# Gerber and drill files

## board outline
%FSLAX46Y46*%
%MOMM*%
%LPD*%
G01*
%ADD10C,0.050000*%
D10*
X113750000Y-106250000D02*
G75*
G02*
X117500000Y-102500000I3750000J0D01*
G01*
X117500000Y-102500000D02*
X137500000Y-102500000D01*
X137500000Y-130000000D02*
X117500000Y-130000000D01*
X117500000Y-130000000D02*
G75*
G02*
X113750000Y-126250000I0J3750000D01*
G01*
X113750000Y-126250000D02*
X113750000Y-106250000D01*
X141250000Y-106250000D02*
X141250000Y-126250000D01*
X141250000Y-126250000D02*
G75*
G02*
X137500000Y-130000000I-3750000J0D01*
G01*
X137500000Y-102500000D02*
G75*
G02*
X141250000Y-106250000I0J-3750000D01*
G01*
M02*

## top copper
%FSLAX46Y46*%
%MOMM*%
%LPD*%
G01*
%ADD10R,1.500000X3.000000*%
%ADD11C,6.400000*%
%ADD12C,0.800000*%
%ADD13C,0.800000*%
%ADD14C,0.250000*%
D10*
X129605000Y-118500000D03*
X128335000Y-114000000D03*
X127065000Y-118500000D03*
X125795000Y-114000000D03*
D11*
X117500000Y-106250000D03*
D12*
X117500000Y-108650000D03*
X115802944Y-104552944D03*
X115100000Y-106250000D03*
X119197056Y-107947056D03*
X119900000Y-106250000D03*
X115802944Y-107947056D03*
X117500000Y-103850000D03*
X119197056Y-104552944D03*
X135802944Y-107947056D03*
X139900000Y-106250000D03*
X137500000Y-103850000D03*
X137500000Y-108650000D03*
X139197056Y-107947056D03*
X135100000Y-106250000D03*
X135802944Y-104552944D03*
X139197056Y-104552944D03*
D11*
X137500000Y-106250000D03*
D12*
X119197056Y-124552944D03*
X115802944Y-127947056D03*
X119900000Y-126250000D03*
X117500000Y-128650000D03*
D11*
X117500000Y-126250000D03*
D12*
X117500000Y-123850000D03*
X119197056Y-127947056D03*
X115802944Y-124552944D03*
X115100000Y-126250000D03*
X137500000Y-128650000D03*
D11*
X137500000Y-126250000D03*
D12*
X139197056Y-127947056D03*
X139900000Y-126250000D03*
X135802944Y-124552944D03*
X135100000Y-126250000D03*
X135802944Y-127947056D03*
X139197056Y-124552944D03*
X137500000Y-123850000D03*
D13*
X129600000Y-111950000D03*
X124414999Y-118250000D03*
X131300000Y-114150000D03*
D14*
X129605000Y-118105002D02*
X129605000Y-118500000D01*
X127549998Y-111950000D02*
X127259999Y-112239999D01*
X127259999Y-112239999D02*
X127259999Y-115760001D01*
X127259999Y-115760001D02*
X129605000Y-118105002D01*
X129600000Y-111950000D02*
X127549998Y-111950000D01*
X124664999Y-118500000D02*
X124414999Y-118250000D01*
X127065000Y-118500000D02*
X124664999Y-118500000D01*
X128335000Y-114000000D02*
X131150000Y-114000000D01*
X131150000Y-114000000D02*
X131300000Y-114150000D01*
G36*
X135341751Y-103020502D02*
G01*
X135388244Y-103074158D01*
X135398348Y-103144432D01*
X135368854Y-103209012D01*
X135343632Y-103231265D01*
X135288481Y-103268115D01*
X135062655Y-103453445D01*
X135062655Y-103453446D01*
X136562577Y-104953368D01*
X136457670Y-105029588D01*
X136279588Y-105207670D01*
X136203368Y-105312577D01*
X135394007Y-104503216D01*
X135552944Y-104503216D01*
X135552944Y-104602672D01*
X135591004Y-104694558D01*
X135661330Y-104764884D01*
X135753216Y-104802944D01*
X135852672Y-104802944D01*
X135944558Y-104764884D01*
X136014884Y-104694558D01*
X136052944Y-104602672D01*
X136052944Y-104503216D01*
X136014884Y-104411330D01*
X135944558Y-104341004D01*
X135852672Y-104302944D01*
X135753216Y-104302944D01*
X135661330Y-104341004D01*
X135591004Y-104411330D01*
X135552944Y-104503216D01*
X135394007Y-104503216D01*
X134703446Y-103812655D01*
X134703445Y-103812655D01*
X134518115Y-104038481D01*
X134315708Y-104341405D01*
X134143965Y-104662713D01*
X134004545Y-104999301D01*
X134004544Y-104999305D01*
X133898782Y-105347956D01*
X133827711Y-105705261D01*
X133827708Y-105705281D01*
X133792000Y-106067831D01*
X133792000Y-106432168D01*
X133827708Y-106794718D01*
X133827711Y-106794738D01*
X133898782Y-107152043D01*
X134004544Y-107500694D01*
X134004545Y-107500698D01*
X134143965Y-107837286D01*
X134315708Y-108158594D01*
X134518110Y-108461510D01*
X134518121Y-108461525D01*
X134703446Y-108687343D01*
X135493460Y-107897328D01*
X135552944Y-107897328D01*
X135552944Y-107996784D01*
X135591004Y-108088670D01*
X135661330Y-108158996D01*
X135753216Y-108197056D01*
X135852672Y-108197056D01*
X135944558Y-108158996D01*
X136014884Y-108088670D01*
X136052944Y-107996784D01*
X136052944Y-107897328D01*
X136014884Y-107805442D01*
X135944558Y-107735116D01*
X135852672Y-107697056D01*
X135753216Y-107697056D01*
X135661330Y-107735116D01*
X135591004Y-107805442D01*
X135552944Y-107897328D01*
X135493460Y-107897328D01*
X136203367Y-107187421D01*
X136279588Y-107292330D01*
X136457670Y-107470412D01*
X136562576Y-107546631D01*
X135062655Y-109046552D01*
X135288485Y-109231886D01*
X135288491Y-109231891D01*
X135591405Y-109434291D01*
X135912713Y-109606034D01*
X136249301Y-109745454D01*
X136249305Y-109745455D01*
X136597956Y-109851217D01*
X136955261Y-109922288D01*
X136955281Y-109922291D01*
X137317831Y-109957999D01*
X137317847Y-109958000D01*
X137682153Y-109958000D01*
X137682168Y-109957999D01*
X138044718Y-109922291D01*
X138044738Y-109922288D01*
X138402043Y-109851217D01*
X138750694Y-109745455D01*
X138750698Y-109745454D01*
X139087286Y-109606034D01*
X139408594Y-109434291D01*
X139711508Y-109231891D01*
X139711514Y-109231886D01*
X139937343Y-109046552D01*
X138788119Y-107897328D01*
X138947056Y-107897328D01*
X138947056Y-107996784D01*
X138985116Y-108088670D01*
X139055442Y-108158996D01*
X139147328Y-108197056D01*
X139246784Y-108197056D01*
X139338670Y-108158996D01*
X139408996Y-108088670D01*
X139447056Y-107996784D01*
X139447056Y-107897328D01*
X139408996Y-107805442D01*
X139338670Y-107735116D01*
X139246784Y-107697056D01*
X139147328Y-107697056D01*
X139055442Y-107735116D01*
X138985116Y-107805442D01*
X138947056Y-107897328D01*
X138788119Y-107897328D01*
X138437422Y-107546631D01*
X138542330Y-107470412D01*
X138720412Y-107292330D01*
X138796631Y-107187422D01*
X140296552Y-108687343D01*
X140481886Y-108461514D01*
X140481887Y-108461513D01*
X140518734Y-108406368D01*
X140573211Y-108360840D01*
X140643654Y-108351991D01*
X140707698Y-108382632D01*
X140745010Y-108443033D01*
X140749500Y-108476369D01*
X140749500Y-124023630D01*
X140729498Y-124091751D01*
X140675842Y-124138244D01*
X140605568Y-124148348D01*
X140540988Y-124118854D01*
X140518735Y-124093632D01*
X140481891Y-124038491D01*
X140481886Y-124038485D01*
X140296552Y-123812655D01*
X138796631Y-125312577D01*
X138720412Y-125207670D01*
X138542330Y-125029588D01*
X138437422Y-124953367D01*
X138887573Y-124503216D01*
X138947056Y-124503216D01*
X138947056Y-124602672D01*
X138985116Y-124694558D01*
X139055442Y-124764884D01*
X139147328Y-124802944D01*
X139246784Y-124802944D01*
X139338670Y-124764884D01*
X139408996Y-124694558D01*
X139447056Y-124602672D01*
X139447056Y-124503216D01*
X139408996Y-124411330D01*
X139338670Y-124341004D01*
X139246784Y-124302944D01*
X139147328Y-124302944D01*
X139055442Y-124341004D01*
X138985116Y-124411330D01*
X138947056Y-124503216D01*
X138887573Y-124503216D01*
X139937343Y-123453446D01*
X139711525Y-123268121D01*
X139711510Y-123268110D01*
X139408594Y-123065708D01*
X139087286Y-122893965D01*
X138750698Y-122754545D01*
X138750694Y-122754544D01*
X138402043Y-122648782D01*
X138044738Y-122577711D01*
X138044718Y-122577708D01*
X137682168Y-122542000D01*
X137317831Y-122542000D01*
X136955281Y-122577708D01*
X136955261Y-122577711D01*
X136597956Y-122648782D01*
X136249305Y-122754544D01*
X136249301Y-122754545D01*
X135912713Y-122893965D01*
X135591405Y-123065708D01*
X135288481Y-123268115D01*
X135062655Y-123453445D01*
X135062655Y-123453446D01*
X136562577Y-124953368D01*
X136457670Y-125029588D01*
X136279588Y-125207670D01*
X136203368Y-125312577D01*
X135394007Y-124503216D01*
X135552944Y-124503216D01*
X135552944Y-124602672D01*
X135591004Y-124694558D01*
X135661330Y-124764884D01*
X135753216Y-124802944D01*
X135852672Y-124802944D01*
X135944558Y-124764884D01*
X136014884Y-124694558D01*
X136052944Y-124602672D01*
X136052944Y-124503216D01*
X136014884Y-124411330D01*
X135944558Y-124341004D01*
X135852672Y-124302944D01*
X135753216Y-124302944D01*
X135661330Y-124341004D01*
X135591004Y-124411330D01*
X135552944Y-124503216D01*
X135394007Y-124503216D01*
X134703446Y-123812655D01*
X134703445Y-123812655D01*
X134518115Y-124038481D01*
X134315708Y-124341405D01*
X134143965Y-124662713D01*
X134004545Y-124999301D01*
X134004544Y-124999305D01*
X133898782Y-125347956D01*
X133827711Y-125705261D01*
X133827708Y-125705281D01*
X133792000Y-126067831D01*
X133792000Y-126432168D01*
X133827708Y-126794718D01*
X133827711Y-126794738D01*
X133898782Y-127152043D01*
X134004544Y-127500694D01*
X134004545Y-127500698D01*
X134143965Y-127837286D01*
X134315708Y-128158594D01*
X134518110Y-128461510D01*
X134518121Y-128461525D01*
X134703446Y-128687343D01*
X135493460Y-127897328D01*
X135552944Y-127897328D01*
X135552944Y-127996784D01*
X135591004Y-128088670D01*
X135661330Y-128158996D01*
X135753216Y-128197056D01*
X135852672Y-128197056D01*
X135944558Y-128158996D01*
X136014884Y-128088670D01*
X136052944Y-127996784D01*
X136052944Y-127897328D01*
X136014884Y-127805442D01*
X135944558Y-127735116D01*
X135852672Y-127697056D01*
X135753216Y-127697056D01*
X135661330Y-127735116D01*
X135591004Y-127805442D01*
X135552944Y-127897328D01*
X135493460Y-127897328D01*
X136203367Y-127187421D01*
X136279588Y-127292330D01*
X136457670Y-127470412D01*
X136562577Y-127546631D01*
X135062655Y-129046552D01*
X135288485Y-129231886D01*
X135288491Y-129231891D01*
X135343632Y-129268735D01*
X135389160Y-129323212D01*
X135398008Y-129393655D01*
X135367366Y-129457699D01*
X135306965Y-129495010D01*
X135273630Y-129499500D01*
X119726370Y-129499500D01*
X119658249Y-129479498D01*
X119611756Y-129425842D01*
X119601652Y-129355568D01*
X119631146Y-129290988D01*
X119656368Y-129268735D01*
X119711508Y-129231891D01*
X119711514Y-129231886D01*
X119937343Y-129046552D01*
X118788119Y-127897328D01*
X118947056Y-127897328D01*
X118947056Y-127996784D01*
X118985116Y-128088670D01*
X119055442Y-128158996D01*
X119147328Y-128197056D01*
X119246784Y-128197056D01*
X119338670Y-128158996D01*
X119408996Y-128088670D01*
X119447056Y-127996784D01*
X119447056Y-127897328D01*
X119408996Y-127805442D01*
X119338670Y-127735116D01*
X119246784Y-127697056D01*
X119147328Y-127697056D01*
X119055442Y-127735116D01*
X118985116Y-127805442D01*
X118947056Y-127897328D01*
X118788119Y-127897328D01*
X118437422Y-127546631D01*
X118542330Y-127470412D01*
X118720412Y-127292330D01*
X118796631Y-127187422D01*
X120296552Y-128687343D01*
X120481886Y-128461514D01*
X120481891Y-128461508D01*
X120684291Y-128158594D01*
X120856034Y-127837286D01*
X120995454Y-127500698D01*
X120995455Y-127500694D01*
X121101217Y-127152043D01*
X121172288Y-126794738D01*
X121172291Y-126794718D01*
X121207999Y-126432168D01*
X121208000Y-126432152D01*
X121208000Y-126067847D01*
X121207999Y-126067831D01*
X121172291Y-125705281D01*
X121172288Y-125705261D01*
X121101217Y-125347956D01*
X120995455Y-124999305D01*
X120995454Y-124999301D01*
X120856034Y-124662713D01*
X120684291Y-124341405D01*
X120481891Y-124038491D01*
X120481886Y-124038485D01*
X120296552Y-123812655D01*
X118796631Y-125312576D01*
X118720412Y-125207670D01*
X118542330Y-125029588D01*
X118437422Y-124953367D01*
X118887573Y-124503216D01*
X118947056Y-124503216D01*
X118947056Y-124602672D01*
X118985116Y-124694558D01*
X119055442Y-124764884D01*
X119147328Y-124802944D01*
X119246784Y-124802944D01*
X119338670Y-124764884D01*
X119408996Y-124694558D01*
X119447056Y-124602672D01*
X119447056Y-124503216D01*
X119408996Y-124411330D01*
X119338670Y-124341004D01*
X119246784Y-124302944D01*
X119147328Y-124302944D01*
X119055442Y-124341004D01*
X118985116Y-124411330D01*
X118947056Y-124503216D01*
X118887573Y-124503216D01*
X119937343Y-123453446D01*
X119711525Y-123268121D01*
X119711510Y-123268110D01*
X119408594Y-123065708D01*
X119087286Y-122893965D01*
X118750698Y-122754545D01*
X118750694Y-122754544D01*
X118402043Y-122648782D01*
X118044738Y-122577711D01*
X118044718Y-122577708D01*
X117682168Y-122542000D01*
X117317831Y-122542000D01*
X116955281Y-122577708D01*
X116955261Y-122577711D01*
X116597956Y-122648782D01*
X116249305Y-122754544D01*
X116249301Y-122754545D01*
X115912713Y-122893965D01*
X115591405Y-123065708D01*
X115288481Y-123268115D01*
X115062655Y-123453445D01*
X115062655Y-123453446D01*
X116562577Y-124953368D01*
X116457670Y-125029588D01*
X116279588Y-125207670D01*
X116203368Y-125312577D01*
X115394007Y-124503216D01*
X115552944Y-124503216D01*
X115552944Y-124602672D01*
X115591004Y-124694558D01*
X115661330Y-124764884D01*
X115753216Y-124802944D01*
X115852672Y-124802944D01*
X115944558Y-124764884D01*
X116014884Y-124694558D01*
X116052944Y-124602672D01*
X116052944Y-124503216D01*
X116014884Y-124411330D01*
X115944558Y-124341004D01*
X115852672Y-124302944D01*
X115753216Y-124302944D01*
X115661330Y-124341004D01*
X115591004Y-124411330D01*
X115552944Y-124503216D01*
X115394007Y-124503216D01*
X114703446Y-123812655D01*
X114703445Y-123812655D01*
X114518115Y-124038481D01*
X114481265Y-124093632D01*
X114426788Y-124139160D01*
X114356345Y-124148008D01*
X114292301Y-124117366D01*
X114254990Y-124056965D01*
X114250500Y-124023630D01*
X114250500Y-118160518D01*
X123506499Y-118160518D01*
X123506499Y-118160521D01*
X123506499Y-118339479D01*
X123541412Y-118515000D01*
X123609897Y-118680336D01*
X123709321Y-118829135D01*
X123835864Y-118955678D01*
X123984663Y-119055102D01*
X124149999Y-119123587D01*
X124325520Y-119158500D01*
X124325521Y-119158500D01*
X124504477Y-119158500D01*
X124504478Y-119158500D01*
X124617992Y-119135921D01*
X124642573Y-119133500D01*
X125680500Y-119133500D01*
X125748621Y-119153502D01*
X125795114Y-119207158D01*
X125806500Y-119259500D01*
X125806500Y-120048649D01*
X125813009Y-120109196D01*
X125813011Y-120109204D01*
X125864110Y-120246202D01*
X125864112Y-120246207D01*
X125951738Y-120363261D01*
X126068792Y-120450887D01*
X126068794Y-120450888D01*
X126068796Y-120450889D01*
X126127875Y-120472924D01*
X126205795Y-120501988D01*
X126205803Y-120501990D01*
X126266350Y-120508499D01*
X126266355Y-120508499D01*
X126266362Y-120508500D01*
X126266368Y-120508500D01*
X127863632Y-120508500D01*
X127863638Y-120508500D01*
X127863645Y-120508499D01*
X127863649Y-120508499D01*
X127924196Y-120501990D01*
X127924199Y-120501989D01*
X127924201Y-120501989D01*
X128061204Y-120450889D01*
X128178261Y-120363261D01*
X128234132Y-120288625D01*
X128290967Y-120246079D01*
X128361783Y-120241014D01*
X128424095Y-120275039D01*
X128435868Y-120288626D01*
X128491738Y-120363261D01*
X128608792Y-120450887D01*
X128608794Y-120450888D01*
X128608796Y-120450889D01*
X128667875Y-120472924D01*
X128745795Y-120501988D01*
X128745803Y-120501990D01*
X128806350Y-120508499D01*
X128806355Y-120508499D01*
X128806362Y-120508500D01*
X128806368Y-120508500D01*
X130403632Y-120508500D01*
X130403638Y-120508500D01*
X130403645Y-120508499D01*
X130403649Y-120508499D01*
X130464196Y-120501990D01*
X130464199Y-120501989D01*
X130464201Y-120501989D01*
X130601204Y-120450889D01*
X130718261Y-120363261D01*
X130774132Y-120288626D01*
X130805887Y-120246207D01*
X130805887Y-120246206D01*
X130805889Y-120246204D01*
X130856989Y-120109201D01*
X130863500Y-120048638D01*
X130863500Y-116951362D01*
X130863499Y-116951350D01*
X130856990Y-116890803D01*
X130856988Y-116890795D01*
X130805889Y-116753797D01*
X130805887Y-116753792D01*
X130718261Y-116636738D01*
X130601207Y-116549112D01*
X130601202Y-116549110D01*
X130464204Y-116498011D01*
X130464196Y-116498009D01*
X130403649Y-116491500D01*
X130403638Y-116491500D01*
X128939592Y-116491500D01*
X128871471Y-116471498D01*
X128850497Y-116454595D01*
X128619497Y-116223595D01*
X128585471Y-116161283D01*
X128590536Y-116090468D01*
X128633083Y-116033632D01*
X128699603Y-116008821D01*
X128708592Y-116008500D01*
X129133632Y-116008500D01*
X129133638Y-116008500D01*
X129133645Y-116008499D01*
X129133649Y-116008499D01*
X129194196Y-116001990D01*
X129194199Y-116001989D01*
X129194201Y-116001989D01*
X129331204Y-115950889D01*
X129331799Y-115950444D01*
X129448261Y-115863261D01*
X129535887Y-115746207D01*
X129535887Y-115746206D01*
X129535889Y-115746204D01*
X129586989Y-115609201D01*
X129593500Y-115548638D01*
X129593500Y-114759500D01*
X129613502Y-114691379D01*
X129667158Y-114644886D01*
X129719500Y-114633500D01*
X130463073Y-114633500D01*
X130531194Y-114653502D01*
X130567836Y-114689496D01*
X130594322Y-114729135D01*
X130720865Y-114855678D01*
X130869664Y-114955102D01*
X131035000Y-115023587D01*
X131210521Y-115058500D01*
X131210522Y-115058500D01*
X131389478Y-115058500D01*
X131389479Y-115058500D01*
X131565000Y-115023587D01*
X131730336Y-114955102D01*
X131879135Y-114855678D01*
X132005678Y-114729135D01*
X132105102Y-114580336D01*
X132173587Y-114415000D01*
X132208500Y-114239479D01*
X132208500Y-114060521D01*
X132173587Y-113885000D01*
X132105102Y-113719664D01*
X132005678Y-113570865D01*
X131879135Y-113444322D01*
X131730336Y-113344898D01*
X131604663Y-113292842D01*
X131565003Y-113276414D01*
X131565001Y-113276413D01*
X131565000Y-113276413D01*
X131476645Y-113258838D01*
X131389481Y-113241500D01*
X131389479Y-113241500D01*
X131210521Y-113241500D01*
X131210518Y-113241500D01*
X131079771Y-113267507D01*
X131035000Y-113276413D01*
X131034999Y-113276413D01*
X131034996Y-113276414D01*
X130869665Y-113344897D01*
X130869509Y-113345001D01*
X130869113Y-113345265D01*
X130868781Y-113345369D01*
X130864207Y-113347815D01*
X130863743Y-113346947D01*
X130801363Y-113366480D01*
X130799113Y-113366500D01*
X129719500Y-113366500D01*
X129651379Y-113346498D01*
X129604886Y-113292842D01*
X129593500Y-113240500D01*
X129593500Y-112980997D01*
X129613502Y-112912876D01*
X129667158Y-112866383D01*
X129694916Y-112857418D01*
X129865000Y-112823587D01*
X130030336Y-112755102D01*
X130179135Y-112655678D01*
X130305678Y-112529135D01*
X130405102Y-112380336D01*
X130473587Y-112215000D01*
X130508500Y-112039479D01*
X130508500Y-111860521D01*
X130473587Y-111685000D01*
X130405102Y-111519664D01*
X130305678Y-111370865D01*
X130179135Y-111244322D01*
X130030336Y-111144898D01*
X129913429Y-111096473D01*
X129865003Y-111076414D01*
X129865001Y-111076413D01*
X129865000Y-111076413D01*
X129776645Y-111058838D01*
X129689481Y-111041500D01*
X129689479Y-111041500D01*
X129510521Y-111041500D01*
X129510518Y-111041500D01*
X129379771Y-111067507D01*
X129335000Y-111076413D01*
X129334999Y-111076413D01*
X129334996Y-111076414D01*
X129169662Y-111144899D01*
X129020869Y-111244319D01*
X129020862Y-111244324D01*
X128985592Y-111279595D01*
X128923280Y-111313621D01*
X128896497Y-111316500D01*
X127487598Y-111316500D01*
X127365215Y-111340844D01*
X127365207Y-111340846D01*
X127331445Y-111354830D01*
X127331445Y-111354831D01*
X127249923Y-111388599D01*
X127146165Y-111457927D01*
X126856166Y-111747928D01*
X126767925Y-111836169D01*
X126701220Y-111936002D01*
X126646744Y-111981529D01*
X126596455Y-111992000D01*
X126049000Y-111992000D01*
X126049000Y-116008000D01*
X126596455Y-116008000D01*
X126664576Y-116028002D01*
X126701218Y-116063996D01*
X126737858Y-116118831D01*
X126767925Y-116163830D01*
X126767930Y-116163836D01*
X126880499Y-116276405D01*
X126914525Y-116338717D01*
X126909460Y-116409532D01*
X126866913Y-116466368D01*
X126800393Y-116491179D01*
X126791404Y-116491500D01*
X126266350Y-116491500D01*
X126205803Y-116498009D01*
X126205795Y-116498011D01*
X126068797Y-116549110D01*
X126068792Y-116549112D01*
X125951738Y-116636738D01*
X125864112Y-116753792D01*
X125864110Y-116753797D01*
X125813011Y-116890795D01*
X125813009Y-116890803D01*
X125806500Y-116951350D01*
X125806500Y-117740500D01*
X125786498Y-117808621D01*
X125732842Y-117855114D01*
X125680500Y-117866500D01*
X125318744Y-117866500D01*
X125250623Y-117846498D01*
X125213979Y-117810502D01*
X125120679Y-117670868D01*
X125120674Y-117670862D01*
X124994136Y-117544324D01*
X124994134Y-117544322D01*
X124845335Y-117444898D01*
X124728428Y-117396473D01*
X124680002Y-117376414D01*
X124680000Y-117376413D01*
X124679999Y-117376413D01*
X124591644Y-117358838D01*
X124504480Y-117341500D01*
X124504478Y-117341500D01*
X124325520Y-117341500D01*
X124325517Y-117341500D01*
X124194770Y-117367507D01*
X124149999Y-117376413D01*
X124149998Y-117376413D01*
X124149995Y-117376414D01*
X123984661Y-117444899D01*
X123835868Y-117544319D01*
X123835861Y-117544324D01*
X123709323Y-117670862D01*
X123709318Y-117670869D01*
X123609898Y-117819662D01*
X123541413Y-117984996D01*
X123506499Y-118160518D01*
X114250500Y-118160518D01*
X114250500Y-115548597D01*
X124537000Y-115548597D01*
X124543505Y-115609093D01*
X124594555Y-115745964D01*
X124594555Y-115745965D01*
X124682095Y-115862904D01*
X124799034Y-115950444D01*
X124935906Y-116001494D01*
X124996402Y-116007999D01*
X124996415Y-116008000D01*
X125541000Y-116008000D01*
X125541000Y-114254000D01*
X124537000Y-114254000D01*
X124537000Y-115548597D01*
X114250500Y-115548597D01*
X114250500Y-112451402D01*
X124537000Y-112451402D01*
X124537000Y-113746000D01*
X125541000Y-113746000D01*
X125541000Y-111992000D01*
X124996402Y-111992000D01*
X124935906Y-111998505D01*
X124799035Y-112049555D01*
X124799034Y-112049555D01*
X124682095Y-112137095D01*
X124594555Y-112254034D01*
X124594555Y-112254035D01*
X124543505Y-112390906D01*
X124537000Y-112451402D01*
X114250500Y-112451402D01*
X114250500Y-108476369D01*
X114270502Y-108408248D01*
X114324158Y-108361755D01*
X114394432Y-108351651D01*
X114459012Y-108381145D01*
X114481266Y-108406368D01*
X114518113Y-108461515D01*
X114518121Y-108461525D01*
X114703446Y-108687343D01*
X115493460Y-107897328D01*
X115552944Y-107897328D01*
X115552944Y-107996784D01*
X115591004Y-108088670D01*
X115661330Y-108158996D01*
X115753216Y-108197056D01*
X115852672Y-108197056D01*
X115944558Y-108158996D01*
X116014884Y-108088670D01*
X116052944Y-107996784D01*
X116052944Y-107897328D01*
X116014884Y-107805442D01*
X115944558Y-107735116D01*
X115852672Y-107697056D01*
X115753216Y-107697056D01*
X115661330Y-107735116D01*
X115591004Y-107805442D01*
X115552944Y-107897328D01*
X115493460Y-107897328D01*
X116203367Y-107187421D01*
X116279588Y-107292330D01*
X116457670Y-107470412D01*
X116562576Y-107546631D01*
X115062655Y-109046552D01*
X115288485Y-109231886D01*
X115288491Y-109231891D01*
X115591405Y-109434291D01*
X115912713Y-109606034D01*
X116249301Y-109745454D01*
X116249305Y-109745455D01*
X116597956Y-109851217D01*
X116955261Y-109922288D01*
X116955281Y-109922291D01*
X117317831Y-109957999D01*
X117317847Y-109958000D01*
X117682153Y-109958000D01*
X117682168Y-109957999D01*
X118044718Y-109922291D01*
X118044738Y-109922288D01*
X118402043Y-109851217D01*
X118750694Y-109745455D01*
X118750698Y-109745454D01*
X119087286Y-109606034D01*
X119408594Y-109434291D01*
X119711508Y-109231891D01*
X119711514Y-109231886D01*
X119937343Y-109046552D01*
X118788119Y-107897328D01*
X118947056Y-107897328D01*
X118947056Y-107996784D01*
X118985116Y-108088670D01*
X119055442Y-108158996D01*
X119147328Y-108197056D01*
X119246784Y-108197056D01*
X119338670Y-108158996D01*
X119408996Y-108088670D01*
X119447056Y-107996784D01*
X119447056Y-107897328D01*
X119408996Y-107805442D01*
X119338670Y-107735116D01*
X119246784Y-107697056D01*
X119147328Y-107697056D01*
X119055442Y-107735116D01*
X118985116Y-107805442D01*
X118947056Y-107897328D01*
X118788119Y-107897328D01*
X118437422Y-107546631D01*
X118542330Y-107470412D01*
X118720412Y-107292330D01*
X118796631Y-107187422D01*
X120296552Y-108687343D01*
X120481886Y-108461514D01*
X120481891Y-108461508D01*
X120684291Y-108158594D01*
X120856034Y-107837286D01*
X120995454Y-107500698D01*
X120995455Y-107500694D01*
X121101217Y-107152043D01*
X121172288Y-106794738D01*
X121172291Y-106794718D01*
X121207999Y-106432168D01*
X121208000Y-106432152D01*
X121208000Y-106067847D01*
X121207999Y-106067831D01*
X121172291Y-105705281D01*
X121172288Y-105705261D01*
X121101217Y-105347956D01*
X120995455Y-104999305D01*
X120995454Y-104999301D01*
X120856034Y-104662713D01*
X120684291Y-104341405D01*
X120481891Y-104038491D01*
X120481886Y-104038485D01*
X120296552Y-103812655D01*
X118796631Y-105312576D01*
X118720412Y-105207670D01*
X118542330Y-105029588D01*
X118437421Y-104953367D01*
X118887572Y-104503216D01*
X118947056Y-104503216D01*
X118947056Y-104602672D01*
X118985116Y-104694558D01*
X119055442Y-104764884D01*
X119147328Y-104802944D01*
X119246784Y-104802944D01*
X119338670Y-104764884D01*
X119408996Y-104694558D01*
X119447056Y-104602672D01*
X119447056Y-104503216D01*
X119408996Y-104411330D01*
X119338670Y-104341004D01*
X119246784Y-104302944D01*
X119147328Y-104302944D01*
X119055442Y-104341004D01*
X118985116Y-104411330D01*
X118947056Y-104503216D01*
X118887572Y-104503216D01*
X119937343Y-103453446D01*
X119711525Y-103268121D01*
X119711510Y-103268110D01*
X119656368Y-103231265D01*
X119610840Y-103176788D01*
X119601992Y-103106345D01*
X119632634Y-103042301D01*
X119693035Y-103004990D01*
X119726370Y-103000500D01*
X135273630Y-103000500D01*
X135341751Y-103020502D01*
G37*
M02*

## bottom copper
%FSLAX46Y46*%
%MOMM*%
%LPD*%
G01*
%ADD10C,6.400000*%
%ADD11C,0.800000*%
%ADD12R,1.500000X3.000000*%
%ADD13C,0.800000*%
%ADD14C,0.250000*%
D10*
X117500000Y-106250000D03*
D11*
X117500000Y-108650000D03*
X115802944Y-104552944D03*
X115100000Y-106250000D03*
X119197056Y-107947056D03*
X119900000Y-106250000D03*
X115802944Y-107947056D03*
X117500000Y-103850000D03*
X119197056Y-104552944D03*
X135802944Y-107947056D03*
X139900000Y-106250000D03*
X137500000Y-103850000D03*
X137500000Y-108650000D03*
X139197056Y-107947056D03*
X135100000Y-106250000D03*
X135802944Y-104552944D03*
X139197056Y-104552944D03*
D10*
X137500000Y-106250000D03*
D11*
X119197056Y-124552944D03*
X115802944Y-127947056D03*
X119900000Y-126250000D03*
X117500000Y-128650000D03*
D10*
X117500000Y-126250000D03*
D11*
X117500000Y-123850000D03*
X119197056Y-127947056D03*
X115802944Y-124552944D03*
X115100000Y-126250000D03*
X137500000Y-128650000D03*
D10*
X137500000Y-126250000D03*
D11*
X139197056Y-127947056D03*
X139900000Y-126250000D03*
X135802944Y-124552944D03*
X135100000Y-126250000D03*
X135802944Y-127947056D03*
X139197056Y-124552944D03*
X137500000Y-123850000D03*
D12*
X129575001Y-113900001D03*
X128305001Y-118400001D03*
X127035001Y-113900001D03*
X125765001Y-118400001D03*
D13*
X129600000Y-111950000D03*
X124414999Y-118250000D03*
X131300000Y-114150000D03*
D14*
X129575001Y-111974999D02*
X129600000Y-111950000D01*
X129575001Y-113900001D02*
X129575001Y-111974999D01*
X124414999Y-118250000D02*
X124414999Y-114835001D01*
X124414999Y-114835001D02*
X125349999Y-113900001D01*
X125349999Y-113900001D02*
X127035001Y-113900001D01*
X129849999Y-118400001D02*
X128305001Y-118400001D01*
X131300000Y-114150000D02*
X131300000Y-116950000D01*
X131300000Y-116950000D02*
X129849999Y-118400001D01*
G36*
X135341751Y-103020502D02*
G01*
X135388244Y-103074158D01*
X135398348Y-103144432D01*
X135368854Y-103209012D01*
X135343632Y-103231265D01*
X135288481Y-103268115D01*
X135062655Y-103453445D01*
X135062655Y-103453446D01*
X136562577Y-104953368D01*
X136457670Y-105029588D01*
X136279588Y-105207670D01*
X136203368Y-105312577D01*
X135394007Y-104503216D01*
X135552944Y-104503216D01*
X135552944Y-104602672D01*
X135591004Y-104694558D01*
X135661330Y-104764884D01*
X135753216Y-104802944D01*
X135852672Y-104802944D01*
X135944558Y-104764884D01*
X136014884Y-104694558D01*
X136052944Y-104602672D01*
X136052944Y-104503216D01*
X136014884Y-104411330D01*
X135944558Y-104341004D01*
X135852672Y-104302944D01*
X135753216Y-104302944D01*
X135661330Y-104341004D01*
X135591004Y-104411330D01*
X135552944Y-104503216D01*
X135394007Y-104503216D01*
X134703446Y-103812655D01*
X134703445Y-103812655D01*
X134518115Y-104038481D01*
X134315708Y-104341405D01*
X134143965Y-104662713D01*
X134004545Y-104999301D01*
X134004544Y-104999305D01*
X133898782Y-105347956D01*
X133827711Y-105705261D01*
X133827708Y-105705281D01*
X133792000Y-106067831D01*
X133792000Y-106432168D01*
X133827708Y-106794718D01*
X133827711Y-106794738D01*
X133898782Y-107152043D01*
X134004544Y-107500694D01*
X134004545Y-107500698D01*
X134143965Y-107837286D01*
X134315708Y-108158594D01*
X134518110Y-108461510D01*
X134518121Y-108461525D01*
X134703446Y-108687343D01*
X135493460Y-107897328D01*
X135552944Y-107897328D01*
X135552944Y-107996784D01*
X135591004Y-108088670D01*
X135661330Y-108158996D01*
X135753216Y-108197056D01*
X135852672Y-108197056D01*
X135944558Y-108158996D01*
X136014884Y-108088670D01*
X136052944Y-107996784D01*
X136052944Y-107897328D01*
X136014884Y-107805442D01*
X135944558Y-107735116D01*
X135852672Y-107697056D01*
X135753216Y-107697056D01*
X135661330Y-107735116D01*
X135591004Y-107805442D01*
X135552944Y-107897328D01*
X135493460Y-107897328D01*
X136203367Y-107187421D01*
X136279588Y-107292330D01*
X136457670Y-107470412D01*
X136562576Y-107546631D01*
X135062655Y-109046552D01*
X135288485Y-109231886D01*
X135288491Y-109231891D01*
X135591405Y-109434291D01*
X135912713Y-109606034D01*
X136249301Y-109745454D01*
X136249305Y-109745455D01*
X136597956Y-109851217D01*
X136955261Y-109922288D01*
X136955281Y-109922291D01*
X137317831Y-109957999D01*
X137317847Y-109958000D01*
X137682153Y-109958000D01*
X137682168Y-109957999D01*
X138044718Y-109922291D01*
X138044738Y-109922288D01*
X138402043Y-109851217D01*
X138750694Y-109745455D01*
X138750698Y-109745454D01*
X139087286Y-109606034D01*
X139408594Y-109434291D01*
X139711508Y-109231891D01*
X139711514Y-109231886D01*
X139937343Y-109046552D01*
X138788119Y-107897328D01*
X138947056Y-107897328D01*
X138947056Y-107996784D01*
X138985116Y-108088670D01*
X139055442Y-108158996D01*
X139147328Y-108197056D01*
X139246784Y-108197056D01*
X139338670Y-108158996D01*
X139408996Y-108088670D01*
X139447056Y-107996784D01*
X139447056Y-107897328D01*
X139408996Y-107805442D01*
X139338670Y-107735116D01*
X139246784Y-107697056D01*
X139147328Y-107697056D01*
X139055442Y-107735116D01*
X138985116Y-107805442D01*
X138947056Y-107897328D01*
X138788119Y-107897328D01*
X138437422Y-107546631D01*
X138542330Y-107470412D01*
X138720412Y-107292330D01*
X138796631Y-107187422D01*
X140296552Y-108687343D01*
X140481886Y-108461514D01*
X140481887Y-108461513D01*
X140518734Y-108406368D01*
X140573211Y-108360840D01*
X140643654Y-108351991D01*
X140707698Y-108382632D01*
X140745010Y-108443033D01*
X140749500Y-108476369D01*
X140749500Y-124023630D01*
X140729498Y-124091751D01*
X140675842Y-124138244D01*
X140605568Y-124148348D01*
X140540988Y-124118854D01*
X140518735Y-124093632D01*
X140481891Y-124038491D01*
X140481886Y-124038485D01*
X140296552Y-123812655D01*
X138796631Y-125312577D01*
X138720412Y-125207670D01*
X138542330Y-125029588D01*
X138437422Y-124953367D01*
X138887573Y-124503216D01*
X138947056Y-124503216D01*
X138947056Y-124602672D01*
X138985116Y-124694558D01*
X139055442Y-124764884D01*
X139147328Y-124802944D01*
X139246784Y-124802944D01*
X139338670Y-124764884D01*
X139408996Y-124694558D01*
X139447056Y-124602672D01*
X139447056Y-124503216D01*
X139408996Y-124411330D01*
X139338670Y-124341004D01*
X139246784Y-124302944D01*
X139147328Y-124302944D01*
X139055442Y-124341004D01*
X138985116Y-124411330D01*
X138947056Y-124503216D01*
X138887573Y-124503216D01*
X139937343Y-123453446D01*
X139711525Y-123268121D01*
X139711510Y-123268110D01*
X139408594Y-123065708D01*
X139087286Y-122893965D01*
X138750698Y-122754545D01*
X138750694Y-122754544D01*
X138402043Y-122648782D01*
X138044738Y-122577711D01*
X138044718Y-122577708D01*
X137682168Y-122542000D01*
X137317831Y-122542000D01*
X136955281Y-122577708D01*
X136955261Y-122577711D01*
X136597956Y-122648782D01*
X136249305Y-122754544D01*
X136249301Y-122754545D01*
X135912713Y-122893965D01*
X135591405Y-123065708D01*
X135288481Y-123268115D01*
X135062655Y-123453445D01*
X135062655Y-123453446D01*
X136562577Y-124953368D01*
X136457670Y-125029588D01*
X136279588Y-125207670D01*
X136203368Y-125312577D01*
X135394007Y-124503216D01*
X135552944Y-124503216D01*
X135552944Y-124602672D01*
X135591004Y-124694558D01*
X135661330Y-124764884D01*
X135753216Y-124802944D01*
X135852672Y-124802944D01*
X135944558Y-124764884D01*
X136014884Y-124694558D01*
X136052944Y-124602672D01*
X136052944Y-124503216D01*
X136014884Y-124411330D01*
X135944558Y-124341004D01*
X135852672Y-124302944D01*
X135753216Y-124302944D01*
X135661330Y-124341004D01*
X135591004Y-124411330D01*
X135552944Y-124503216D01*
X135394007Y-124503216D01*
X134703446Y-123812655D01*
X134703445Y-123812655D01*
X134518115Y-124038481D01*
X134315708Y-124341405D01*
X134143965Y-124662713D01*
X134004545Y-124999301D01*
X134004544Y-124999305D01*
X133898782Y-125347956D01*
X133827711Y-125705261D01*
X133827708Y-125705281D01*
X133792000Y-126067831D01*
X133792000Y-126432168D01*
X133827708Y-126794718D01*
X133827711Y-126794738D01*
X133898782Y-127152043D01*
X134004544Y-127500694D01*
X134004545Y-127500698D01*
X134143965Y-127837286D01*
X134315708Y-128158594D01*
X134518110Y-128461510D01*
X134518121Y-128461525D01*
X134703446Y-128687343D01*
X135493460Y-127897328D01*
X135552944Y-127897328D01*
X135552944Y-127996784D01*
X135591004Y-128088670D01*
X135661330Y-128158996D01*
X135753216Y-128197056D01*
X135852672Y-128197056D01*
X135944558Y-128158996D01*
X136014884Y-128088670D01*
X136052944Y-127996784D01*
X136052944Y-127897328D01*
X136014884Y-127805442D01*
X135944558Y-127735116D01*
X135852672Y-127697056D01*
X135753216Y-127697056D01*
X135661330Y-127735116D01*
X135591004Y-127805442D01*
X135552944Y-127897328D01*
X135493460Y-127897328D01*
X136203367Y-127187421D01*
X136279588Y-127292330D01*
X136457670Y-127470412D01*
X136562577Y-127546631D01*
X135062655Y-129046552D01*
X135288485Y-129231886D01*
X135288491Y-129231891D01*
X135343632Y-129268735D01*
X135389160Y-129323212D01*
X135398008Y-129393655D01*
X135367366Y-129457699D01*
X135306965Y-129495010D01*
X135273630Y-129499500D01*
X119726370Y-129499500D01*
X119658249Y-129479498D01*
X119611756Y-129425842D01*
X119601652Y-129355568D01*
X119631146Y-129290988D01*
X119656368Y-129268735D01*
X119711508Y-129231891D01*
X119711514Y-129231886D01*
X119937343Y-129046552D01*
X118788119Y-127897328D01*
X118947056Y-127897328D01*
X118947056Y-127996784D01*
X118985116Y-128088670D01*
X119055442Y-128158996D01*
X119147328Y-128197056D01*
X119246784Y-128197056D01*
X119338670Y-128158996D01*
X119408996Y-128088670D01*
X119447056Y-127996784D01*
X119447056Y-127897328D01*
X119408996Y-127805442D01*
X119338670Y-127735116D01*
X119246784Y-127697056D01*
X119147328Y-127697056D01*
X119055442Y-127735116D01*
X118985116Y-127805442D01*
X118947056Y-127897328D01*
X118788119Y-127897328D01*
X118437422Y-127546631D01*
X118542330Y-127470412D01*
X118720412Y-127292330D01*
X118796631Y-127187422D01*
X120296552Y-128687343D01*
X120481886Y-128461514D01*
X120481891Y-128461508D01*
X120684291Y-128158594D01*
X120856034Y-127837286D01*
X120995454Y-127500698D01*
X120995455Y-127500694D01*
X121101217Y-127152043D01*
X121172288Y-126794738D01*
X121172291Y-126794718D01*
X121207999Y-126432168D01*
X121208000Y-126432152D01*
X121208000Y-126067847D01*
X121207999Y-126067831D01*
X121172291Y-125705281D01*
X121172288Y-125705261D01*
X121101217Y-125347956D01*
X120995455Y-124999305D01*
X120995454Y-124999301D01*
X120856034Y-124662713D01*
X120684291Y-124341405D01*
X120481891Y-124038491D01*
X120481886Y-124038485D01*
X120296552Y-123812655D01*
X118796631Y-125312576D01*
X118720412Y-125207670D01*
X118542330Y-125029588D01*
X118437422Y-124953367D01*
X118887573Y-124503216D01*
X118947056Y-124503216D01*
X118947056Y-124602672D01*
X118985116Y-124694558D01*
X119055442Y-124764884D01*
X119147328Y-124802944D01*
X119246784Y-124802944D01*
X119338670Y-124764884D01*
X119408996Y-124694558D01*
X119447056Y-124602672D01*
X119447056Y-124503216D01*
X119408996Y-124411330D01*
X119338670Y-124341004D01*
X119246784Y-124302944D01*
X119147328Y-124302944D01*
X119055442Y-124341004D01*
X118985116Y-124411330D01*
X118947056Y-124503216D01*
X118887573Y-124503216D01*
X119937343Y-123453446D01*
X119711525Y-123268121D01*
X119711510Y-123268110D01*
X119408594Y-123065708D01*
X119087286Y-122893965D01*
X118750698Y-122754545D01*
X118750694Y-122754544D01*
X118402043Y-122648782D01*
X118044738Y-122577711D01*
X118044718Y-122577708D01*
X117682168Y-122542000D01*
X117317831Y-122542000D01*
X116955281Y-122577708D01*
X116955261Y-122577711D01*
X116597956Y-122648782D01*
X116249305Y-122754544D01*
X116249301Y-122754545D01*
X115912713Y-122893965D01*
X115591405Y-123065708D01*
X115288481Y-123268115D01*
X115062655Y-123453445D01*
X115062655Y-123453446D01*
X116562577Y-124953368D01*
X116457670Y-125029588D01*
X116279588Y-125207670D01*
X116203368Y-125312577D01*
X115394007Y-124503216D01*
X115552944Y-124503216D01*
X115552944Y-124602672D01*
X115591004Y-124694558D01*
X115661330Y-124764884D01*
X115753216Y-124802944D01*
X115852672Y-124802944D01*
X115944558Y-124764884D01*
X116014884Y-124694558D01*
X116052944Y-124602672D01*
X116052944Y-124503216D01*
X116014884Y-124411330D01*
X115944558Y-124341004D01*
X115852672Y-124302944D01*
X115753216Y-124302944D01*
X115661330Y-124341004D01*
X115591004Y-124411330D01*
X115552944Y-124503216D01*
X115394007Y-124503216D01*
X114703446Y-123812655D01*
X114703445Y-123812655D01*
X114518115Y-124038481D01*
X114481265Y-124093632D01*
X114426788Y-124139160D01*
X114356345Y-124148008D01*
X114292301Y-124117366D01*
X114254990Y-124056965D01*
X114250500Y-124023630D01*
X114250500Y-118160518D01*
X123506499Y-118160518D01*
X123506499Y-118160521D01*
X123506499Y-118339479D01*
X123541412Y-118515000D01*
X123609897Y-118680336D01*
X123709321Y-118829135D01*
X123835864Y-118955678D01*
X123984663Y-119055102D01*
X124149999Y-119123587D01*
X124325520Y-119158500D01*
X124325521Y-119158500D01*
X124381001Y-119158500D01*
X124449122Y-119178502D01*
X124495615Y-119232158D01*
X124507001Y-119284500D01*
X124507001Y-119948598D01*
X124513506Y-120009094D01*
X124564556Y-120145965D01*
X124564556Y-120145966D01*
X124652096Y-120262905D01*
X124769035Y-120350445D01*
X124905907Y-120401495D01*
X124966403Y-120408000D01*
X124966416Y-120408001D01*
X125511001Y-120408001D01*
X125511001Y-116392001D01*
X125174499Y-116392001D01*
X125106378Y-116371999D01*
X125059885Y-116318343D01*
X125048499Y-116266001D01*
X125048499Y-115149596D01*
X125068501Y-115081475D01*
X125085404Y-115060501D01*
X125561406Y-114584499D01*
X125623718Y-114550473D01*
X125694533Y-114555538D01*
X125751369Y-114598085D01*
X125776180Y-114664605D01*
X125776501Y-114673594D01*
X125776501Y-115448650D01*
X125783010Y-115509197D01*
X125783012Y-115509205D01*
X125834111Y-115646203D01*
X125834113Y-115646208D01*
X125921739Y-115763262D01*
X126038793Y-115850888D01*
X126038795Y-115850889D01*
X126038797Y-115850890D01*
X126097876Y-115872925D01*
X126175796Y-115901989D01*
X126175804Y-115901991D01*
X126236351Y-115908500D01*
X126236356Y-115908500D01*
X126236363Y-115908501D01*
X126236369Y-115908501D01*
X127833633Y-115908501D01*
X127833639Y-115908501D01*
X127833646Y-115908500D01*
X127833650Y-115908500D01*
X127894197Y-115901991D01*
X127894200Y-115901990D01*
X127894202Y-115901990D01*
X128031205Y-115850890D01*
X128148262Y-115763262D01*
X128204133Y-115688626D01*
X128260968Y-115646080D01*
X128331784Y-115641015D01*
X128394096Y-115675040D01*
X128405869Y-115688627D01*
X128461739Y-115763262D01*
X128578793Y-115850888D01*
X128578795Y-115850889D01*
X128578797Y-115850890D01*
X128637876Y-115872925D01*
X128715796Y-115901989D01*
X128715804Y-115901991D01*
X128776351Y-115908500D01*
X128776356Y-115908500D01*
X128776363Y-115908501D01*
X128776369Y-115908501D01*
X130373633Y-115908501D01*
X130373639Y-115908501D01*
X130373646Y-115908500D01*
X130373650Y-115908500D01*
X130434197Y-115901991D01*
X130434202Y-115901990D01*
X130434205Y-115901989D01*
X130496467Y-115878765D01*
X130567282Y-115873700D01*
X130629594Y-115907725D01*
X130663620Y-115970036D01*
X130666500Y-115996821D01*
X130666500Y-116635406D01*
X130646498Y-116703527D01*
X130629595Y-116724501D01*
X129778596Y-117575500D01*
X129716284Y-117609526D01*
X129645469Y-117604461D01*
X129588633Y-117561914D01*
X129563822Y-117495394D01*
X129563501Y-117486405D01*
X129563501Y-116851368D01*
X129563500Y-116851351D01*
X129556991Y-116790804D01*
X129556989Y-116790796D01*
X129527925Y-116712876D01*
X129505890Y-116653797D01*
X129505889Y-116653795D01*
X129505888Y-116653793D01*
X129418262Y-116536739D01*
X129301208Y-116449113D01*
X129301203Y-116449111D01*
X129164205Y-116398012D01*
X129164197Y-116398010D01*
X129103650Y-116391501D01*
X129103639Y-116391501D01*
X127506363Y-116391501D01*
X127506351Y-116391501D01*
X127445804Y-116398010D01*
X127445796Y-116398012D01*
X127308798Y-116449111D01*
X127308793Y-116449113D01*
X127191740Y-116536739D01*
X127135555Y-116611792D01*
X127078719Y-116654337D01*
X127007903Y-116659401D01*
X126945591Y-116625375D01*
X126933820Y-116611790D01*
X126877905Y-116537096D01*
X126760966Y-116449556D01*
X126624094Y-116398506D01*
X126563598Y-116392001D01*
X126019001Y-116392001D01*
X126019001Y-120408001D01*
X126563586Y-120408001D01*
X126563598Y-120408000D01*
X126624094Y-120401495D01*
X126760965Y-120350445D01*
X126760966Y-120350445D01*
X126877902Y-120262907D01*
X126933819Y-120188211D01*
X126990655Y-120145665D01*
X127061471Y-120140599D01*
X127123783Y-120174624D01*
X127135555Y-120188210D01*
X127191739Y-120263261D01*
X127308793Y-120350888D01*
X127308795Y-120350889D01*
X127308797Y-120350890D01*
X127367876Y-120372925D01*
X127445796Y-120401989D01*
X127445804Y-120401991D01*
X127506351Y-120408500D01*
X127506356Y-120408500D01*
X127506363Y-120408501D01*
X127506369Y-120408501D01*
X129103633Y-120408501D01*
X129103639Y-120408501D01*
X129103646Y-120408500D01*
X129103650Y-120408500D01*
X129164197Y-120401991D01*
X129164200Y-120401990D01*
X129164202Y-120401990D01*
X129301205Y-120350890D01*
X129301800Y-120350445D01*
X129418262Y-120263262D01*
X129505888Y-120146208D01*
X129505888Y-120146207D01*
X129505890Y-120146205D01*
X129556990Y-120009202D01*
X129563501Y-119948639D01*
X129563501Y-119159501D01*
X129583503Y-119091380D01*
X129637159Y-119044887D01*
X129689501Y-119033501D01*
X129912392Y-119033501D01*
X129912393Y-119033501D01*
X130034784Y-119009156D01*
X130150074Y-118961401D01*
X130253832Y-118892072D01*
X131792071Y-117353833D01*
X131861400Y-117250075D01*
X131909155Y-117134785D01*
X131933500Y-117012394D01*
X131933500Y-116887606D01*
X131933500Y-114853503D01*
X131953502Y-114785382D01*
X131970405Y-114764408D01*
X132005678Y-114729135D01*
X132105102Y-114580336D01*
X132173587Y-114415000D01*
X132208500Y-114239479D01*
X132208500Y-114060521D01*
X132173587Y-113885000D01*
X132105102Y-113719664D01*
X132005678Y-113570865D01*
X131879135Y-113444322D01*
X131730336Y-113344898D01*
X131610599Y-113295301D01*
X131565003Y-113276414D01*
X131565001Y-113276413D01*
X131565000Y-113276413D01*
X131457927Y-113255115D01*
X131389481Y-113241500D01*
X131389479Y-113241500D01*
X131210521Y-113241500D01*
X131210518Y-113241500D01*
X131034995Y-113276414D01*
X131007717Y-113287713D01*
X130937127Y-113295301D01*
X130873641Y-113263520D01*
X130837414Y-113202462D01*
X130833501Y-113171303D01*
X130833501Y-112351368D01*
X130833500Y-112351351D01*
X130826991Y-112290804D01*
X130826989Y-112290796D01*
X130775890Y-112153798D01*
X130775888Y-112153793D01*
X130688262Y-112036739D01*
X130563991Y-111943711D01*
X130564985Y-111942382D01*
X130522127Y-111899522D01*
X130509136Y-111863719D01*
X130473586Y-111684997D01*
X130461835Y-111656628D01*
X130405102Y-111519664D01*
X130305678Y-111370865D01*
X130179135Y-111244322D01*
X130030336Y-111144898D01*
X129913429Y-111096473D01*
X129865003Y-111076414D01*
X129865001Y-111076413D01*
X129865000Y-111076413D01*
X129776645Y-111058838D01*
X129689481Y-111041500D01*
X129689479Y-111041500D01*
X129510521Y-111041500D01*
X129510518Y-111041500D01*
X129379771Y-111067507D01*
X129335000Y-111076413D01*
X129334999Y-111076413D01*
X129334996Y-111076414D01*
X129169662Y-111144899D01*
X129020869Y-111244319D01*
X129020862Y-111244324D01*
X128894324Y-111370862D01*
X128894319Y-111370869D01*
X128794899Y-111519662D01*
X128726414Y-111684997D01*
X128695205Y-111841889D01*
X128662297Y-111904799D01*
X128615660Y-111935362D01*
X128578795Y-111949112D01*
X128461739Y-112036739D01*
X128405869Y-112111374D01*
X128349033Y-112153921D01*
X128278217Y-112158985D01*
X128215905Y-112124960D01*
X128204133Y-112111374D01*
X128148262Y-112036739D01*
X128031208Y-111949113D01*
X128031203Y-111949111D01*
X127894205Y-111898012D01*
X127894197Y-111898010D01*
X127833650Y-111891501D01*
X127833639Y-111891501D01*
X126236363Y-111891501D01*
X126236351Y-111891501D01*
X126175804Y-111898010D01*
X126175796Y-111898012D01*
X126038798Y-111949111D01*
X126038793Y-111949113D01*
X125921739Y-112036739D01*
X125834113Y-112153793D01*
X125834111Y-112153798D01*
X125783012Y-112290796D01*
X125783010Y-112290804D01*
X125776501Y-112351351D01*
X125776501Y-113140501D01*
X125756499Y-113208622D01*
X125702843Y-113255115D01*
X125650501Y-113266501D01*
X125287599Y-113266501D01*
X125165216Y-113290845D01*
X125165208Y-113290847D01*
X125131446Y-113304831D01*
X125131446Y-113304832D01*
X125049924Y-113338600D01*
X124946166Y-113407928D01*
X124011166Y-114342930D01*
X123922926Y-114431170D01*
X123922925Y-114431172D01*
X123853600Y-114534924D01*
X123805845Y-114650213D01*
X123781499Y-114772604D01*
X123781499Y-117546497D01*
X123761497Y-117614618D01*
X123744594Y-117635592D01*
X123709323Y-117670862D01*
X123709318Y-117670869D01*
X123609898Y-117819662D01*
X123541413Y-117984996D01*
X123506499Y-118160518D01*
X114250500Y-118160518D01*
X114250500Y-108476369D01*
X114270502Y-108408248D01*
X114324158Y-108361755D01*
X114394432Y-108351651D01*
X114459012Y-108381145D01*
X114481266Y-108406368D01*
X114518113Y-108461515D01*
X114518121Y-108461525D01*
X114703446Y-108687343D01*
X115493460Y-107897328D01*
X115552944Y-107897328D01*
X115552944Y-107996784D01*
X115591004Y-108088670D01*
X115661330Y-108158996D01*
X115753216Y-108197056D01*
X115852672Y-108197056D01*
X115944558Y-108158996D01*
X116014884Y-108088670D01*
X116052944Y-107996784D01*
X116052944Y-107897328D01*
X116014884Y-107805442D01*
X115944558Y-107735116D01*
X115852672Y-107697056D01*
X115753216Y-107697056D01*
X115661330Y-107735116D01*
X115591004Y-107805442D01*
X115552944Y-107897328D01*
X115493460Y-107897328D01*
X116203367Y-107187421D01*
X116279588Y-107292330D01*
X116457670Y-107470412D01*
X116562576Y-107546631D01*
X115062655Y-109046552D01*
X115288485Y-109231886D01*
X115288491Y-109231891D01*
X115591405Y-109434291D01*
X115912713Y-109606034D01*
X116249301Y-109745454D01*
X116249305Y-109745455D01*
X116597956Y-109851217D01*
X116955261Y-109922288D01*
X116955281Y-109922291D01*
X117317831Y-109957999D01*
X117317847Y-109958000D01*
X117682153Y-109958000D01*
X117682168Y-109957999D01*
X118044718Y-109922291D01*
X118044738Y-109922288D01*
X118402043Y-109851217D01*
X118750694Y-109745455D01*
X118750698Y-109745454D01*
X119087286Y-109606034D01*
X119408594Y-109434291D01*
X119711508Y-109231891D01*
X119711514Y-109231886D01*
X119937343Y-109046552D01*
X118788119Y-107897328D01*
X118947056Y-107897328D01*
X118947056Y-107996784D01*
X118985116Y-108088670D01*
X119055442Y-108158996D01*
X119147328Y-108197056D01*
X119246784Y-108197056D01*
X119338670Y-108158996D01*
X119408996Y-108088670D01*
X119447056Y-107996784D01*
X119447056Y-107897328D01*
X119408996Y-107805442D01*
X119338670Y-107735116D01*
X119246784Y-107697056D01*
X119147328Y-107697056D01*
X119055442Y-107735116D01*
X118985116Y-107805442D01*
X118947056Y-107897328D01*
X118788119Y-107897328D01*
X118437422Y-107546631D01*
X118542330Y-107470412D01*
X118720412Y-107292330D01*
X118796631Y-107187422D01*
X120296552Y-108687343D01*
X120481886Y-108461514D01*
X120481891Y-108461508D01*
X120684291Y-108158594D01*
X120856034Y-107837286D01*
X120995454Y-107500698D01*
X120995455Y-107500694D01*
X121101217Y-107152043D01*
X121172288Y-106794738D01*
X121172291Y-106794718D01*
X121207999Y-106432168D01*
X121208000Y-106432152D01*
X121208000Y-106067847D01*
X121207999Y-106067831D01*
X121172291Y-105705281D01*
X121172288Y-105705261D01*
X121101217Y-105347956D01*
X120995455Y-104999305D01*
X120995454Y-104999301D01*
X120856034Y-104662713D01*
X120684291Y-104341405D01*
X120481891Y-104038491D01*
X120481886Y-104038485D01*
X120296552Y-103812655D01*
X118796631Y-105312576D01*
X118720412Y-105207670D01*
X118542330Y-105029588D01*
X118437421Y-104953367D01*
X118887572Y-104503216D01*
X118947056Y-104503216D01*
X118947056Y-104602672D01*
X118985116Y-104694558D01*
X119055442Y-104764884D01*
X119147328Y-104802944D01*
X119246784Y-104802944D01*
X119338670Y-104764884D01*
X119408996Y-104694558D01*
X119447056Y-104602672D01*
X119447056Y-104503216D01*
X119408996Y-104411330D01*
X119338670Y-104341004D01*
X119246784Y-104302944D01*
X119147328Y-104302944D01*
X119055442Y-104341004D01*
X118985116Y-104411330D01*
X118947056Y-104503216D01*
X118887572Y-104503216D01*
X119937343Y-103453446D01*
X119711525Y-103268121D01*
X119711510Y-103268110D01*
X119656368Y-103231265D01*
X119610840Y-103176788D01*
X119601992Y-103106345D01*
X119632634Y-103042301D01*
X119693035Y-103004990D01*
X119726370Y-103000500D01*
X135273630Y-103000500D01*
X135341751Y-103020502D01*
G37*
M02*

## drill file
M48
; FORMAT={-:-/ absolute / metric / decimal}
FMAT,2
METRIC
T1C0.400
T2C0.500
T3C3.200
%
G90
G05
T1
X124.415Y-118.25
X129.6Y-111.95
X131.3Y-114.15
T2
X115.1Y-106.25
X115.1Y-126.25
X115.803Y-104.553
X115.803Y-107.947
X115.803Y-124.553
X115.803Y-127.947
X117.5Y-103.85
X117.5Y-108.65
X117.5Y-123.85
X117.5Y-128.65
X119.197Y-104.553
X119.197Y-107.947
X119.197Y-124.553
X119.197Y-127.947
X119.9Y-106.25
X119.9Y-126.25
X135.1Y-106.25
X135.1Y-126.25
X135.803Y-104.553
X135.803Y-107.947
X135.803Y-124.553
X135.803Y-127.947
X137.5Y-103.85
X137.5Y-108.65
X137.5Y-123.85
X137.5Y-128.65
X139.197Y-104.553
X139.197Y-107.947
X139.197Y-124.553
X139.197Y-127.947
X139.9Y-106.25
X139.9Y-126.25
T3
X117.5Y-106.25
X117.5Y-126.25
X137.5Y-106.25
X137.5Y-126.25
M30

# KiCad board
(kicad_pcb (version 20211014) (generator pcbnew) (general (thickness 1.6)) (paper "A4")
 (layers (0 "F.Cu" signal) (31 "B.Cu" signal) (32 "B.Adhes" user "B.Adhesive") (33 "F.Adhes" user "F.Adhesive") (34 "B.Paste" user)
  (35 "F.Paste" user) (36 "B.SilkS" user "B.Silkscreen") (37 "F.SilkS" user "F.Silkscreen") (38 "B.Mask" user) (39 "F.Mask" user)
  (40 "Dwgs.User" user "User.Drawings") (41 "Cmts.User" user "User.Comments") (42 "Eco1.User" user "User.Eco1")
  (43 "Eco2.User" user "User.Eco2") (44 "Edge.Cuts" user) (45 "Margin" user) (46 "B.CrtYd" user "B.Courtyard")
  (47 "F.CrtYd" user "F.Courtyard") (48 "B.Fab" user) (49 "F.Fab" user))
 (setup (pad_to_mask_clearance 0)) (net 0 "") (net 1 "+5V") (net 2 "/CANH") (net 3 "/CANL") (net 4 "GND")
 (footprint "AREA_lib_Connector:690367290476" (layer "F.Cu") (at 127.7 116.25)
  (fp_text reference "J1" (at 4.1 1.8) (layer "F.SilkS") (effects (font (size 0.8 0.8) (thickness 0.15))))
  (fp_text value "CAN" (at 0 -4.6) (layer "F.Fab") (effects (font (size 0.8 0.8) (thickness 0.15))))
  (pad "1" smd rect locked (at 1.905 2.25) (size 1.5 3) (layers "F.Cu" "F.Paste" "F.Mask") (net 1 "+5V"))
  (pad "2" smd rect locked (at 0.635 -2.25) (size 1.5 3) (layers "F.Cu" "F.Paste" "F.Mask") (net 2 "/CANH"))
  (pad "3" smd rect locked (at -0.635 2.25) (size 1.5 3) (layers "F.Cu" "F.Paste" "F.Mask") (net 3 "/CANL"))
  (pad "4" smd rect locked (at -1.905 -2.25) (size 1.5 3) (layers "F.Cu" "F.Paste" "F.Mask") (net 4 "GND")))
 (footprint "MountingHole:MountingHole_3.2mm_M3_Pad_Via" (layer "F.Cu") (at 117.5 106.25)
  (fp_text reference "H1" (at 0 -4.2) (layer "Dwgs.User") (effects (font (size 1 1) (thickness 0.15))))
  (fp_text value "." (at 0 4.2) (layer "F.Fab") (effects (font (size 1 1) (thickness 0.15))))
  (pad "1" thru_hole circle locked (at 0 0) (size 6.4 6.4) (drill 3.2) (layers *.Cu *.Mask) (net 4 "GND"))
  (pad "1" thru_hole circle locked (at 0 2.4) (size 0.8 0.8) (drill 0.5) (layers *.Cu *.Mask) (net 4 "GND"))
  (pad "1" thru_hole circle locked (at -1.697056 -1.697056) (size 0.8 0.8) (drill 0.5) (layers *.Cu *.Mask) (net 4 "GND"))
  (pad "1" thru_hole circle locked (at -2.4 0) (size 0.8 0.8) (drill 0.5) (layers *.Cu *.Mask) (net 4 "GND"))
  (pad "1" thru_hole circle locked (at 1.697056 1.697056) (size 0.8 0.8) (drill 0.5) (layers *.Cu *.Mask) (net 4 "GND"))
  (pad "1" thru_hole circle locked (at 2.4 0) (size 0.8 0.8) (drill 0.5) (layers *.Cu *.Mask) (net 4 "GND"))
  (pad "1" thru_hole circle locked (at -1.697056 1.697056) (size 0.8 0.8) (drill 0.5) (layers *.Cu *.Mask) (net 4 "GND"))
  (pad "1" thru_hole circle locked (at 0 -2.4) (size 0.8 0.8) (drill 0.5) (layers *.Cu *.Mask) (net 4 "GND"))
  (pad "1" thru_hole circle locked (at 1.697056 -1.697056) (size 0.8 0.8) (drill 0.5) (layers *.Cu *.Mask) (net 4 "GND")))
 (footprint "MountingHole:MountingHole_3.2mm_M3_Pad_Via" (layer "F.Cu") (at 137.5 106.25)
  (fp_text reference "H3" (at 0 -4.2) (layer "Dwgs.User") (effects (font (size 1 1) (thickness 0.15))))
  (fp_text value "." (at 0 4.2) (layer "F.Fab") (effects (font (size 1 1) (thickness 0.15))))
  (pad "1" thru_hole circle locked (at -1.697056 1.697056) (size 0.8 0.8) (drill 0.5) (layers *.Cu *.Mask) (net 4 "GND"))
  (pad "1" thru_hole circle locked (at 2.4 0) (size 0.8 0.8) (drill 0.5) (layers *.Cu *.Mask) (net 4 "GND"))
  (pad "1" thru_hole circle locked (at 0 -2.4) (size 0.8 0.8) (drill 0.5) (layers *.Cu *.Mask) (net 4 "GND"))
  (pad "1" thru_hole circle locked (at 0 2.4) (size 0.8 0.8) (drill 0.5) (layers *.Cu *.Mask) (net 4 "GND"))
  (pad "1" thru_hole circle locked (at 1.697056 1.697056) (size 0.8 0.8) (drill 0.5) (layers *.Cu *.Mask) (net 4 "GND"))
  (pad "1" thru_hole circle locked (at -2.4 0) (size 0.8 0.8) (drill 0.5) (layers *.Cu *.Mask) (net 4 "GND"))
  (pad "1" thru_hole circle locked (at -1.697056 -1.697056) (size 0.8 0.8) (drill 0.5) (layers *.Cu *.Mask) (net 4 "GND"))
  (pad "1" thru_hole circle locked (at 1.697056 -1.697056) (size 0.8 0.8) (drill 0.5) (layers *.Cu *.Mask) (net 4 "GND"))
  (pad "1" thru_hole circle locked (at 0 0) (size 6.4 6.4) (drill 3.2) (layers *.Cu *.Mask) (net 4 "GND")))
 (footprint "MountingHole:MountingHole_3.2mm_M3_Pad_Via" (layer "F.Cu") (at 117.5 126.25)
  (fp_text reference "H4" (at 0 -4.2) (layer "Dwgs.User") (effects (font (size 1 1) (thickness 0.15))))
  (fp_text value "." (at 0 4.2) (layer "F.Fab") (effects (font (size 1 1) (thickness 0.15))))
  (pad "1" thru_hole circle locked (at 1.697056 -1.697056) (size 0.8 0.8) (drill 0.5) (layers *.Cu *.Mask) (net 4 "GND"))
  (pad "1" thru_hole circle locked (at -1.697056 1.697056) (size 0.8 0.8) (drill 0.5) (layers *.Cu *.Mask) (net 4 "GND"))
  (pad "1" thru_hole circle locked (at 2.4 0) (size 0.8 0.8) (drill 0.5) (layers *.Cu *.Mask) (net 4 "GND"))
  (pad "1" thru_hole circle locked (at 0 2.4) (size 0.8 0.8) (drill 0.5) (layers *.Cu *.Mask) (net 4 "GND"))
  (pad "1" thru_hole circle locked (at 0 0) (size 6.4 6.4) (drill 3.2) (layers *.Cu *.Mask) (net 4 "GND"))
  (pad "1" thru_hole circle locked (at 0 -2.4) (size 0.8 0.8) (drill 0.5) (layers *.Cu *.Mask) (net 4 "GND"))
  (pad "1" thru_hole circle locked (at 1.697056 1.697056) (size 0.8 0.8) (drill 0.5) (layers *.Cu *.Mask) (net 4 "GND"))
  (pad "1" thru_hole circle locked (at -1.697056 -1.697056) (size 0.8 0.8) (drill 0.5) (layers *.Cu *.Mask) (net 4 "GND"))
  (pad "1" thru_hole circle locked (at -2.4 0) (size 0.8 0.8) (drill 0.5) (layers *.Cu *.Mask) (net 4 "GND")))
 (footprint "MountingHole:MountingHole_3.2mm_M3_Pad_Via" (layer "F.Cu") (at 137.5 126.25)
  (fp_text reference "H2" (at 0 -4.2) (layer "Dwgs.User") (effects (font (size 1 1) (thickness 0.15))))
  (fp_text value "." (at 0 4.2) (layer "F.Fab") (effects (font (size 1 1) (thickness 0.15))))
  (pad "1" thru_hole circle locked (at 0 2.4) (size 0.8 0.8) (drill 0.5) (layers *.Cu *.Mask) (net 4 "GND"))
  (pad "1" thru_hole circle locked (at 0 0) (size 6.4 6.4) (drill 3.2) (layers *.Cu *.Mask) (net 4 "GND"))
  (pad "1" thru_hole circle locked (at 1.697056 1.697056) (size 0.8 0.8) (drill 0.5) (layers *.Cu *.Mask) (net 4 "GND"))
  (pad "1" thru_hole circle locked (at 2.4 0) (size 0.8 0.8) (drill 0.5) (layers *.Cu *.Mask) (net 4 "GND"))
  (pad "1" thru_hole circle locked (at -1.697056 -1.697056) (size 0.8 0.8) (drill 0.5) (layers *.Cu *.Mask) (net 4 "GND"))
  (pad "1" thru_hole circle locked (at -2.4 0) (size 0.8 0.8) (drill 0.5) (layers *.Cu *.Mask) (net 4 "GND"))
  (pad "1" thru_hole circle locked (at -1.697056 1.697056) (size 0.8 0.8) (drill 0.5) (layers *.Cu *.Mask) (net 4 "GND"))
  (pad "1" thru_hole circle locked (at 1.697056 -1.697056) (size 0.8 0.8) (drill 0.5) (layers *.Cu *.Mask) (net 4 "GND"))
  (pad "1" thru_hole circle locked (at 0 -2.4) (size 0.8 0.8) (drill 0.5) (layers *.Cu *.Mask) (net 4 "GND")))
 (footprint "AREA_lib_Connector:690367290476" (layer "B.Cu") (at 127.670001 116.150001)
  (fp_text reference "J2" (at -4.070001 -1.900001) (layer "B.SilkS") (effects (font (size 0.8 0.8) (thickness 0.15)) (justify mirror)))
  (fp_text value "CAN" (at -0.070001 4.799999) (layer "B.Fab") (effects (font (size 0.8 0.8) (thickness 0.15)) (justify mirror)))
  (pad "1" smd rect locked (at 1.905 -2.25) (size 1.5 3) (layers "B.Cu" "B.Paste" "B.Mask") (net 1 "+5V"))
  (pad "2" smd rect locked (at 0.635 2.25) (size 1.5 3) (layers "B.Cu" "B.Paste" "B.Mask") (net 2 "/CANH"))
  (pad "3" smd rect locked (at -0.635 -2.25) (size 1.5 3) (layers "B.Cu" "B.Paste" "B.Mask") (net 3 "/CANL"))
  (pad "4" smd rect locked (at -1.905 2.25) (size 1.5 3) (layers "B.Cu" "B.Paste" "B.Mask") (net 4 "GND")))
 (gr_arc (start 113.75 106.25) (mid 114.84835 103.59835) (end 117.5 102.5) (layer "Edge.Cuts") (width 0.05))
 (gr_line (start 117.5 102.5) (end 137.5 102.5) (layer "Edge.Cuts") (width 0.05))
 (gr_line (start 137.5 130) (end 117.5 130) (layer "Edge.Cuts") (width 0.05))
 (gr_arc (start 117.5 130) (mid 114.84835 128.90165) (end 113.75 126.25) (layer "Edge.Cuts") (width 0.05))
 (gr_line (start 113.75 126.25) (end 113.75 106.25) (layer "Edge.Cuts") (width 0.05))
 (gr_line (start 141.25 106.25) (end 141.25 126.25) (layer "Edge.Cuts") (width 0.05))
 (gr_arc (start 141.25 126.25) (mid 140.15165 128.90165) (end 137.5 130) (layer "Edge.Cuts") (width 0.05))
 (gr_arc (start 137.5 102.5) (mid 140.15165 103.59835) (end 141.25 106.25) (layer "Edge.Cuts") (width 0.05))
 (segment (start 129.605 118.105002) (end 129.605 118.5) (width 0.25) (layer "F.Cu") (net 1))
 (segment (start 127.549998 111.95) (end 127.259999 112.239999) (width 0.25) (layer "F.Cu") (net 1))
 (segment (start 127.259999 112.239999) (end 127.259999 115.760001) (width 0.25) (layer "F.Cu") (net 1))
 (segment (start 127.259999 115.760001) (end 129.605 118.105002) (width 0.25) (layer "F.Cu") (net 1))
 (segment (start 129.6 111.95) (end 127.549998 111.95) (width 0.25) (layer "F.Cu") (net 1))
 (via (at 129.6 111.95) (size 0.8) (drill 0.4) (layers "F.Cu" "B.Cu") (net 1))
 (segment (start 129.575001 111.974999) (end 129.6 111.95) (width 0.25) (layer "B.Cu") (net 1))
 (segment (start 129.575001 113.900001) (end 129.575001 111.974999) (width 0.25) (layer "B.Cu") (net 1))
 (segment (start 124.664999 118.5) (end 124.414999 118.25) (width 0.25) (layer "F.Cu") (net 3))
 (segment (start 127.065 118.5) (end 124.664999 118.5) (width 0.25) (layer "F.Cu") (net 3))
 (via (at 124.414999 118.25) (size 0.8) (drill 0.4) (layers "F.Cu" "B.Cu") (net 3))
 (segment (start 124.414999 118.25) (end 124.414999 114.835001) (width 0.25) (layer "B.Cu") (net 3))
 (segment (start 124.414999 114.835001) (end 125.349999 113.900001) (width 0.25) (layer "B.Cu") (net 3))
 (segment (start 125.349999 113.900001) (end 127.035001 113.900001) (width 0.25) (layer "B.Cu") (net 3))
 (segment (start 128.335 114) (end 131.15 114) (width 0.25) (layer "F.Cu") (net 2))
 (segment (start 131.15 114) (end 131.3 114.15) (width 0.25) (layer "F.Cu") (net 2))
 (via (at 131.3 114.15) (size 0.8) (drill 0.4) (layers "F.Cu" "B.Cu") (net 2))
 (segment (start 129.849999 118.400001) (end 128.305001 118.400001) (width 0.25) (layer "B.Cu") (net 2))
 (segment (start 131.3 114.15) (end 131.3 116.95) (width 0.25) (layer "B.Cu") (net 2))
 (segment (start 131.3 116.95) (end 129.849999 118.400001) (width 0.25) (layer "B.Cu") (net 2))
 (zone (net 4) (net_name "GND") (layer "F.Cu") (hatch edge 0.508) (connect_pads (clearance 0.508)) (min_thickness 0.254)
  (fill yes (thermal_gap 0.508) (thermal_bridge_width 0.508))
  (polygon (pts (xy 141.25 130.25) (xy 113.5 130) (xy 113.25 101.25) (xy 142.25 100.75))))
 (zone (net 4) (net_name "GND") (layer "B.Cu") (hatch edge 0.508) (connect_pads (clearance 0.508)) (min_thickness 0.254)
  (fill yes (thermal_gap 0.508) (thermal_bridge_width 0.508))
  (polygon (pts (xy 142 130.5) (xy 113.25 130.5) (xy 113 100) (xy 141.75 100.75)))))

